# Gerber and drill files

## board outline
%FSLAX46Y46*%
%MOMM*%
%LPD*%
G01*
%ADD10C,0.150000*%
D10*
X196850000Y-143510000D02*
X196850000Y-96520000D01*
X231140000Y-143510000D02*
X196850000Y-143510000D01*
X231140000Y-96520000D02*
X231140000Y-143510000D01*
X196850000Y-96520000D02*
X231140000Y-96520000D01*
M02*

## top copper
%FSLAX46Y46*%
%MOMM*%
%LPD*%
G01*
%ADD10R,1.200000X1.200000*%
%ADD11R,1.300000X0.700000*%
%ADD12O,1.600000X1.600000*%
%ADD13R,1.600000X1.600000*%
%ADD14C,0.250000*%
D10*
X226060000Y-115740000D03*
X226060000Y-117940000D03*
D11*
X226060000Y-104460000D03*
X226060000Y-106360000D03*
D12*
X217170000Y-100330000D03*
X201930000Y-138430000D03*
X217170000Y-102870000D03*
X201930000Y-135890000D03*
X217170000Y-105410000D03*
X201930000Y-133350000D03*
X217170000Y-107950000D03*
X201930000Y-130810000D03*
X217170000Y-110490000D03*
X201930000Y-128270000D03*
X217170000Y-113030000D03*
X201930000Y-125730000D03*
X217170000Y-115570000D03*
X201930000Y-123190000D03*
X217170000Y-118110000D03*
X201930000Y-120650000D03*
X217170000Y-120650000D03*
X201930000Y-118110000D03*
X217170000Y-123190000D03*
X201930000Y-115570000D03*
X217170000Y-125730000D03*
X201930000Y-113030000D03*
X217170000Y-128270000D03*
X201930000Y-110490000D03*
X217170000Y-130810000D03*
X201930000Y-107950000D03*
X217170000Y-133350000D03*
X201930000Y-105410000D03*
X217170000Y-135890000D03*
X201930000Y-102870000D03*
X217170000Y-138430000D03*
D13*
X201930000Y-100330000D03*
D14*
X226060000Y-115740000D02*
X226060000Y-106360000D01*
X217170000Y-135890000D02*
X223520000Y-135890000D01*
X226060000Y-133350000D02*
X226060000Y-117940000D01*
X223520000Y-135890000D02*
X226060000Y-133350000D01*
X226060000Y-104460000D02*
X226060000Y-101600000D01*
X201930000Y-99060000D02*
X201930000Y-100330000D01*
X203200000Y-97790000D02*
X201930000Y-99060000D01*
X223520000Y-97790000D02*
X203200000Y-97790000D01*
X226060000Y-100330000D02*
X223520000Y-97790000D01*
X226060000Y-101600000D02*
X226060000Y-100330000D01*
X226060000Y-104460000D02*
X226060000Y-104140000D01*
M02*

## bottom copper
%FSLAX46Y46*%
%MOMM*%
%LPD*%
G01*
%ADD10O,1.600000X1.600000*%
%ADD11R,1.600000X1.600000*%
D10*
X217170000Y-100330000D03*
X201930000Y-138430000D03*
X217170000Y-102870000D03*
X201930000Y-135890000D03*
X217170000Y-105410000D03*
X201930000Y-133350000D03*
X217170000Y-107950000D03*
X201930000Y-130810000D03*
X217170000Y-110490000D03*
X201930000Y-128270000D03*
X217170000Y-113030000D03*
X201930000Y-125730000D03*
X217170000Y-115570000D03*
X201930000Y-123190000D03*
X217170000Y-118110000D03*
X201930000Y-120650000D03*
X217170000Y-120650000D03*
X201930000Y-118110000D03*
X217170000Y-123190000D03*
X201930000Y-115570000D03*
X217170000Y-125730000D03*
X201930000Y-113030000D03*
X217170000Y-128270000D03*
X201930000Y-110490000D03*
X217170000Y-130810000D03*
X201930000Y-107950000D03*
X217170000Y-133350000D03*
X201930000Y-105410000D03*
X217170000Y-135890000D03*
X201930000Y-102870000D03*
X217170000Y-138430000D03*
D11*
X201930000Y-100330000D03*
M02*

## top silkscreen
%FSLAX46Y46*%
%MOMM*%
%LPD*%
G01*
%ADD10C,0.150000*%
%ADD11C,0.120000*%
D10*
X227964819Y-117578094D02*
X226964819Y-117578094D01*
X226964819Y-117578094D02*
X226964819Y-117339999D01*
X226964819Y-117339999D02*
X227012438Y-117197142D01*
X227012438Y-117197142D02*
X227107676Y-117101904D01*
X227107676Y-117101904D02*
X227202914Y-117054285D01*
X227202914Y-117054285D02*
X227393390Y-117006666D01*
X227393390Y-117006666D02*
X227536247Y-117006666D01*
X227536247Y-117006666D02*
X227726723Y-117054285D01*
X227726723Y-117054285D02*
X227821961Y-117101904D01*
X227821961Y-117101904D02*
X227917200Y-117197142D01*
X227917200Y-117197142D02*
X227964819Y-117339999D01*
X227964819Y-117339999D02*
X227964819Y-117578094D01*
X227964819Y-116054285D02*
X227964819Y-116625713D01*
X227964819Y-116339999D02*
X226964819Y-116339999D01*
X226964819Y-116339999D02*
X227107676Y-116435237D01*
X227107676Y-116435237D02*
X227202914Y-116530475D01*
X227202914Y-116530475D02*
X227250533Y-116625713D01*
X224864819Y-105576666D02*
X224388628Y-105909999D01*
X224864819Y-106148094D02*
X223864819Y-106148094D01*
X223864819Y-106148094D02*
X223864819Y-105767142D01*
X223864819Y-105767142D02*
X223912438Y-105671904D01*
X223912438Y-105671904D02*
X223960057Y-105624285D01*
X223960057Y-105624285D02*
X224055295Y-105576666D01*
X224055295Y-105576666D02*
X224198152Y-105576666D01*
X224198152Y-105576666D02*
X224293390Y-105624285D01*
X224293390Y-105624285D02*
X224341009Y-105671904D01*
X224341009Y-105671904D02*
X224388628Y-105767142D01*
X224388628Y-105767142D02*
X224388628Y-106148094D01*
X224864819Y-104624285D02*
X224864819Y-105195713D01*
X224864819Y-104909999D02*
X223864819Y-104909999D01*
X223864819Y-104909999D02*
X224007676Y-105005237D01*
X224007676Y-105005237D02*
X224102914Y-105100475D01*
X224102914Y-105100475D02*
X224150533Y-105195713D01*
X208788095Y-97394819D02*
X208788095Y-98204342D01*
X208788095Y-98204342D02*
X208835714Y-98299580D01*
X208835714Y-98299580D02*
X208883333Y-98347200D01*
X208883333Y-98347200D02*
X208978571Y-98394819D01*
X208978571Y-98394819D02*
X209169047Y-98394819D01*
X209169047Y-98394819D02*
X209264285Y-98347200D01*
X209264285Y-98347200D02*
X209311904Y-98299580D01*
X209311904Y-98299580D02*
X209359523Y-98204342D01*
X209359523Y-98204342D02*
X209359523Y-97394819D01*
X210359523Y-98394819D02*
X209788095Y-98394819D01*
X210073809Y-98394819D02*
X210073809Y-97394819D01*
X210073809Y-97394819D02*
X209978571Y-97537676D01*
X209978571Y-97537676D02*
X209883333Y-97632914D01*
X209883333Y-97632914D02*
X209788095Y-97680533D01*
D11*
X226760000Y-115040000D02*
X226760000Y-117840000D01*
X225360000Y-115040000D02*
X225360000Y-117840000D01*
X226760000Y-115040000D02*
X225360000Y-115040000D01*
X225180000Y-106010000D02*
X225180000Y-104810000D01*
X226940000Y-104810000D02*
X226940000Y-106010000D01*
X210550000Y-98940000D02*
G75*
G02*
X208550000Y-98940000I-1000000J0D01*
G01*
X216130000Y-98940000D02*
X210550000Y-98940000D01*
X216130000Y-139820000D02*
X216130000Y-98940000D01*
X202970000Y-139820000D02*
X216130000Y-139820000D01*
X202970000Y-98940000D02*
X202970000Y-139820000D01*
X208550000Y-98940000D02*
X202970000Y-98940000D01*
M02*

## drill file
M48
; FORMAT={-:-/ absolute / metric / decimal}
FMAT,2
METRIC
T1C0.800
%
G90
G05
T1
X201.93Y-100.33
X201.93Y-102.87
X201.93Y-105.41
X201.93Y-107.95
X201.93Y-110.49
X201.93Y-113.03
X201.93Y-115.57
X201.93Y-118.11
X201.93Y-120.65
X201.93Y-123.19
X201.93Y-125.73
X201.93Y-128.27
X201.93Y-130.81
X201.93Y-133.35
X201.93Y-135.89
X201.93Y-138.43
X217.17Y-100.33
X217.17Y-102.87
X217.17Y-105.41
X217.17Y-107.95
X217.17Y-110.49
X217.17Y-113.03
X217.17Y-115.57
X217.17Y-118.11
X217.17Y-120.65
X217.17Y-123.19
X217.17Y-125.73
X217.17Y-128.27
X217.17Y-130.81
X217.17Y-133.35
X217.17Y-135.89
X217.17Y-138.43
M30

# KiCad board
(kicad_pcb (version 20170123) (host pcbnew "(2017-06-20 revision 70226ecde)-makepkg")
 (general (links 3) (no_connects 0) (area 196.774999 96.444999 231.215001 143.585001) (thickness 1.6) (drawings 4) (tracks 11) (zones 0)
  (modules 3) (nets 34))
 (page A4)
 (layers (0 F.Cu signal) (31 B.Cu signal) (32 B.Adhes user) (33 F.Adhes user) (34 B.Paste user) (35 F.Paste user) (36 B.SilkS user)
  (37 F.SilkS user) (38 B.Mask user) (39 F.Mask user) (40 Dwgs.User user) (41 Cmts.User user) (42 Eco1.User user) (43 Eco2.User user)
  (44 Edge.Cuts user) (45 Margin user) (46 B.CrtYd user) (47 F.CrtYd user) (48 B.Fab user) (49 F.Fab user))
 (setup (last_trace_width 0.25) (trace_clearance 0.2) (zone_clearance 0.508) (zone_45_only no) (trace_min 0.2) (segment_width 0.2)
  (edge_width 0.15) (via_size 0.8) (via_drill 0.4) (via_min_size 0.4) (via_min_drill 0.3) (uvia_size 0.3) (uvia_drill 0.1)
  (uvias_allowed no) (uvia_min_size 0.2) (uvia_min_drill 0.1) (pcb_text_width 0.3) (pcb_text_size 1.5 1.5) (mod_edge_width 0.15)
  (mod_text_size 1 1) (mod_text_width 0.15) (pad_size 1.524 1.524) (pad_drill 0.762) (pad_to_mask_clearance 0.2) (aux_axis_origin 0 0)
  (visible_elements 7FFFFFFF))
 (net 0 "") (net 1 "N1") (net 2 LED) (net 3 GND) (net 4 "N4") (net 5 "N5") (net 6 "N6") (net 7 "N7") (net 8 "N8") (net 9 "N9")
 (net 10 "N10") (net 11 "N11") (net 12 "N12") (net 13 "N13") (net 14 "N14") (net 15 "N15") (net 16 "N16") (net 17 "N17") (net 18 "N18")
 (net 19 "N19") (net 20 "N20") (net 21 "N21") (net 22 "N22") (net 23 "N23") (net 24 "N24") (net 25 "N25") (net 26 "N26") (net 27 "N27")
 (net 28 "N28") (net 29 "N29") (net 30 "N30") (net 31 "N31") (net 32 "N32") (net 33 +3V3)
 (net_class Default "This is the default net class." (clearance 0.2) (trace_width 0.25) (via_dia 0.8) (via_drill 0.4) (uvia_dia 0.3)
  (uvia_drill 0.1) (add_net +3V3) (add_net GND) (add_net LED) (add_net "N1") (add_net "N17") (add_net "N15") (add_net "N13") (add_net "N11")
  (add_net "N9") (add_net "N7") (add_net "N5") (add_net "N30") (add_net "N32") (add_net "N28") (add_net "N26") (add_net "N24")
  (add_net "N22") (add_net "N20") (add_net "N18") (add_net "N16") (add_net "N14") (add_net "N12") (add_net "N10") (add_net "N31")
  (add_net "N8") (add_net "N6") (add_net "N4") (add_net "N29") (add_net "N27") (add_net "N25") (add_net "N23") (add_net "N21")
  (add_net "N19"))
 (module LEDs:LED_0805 (layer F.Cu) (at 226.06 116.84 270)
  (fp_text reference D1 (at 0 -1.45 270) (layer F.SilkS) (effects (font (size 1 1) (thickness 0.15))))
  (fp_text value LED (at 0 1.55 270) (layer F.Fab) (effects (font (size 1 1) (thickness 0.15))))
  (fp_line (start -1.8 -0.7) (end 1 -0.7) (layer F.SilkS) (width 0.12))
  (fp_line (start -1.8 0.7) (end 1 0.7) (layer F.SilkS) (width 0.12))
  (fp_line (start -1.8 -0.7) (end -1.8 0.7) (layer F.SilkS) (width 0.12))
  (pad 1 smd rect (at -1.1 0 90) (size 1.2 1.2) (layers F.Cu F.Paste F.Mask) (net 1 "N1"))
  (pad 2 smd rect (at 1.1 0 90) (size 1.2 1.2) (layers F.Cu F.Paste F.Mask) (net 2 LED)))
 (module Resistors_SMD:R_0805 (layer F.Cu) (at 226.06 105.41 90)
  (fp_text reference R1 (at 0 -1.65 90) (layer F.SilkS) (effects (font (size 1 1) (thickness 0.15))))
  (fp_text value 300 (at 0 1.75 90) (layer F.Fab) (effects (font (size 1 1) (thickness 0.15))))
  (fp_line (start -0.6 -0.88) (end 0.6 -0.88) (layer F.SilkS) (width 0.12))
  (fp_line (start 0.6 0.88) (end -0.6 0.88) (layer F.SilkS) (width 0.12))
  (pad 2 smd rect (at 0.95 0 90) (size 0.7 1.3) (layers F.Cu F.Paste F.Mask) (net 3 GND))
  (pad 1 smd rect (at -0.95 0 90) (size 0.7 1.3) (layers F.Cu F.Paste F.Mask) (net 1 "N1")))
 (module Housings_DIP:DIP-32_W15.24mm (layer F.Cu) (at 201.93 100.33)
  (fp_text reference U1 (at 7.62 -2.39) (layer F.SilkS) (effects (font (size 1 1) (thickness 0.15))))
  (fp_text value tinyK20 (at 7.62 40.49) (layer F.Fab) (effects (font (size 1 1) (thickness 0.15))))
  (fp_arc (start 7.62 -1.39) (end 6.62 -1.39) (angle -180) (layer F.SilkS) (width 0.12))
  (fp_line (start 14.2 -1.39) (end 8.62 -1.39) (layer F.SilkS) (width 0.12))
  (fp_line (start 14.2 39.49) (end 14.2 -1.39) (layer F.SilkS) (width 0.12))
  (fp_line (start 1.04 39.49) (end 14.2 39.49) (layer F.SilkS) (width 0.12))
  (fp_line (start 1.04 -1.39) (end 1.04 39.49) (layer F.SilkS) (width 0.12))
  (fp_line (start 6.62 -1.39) (end 1.04 -1.39) (layer F.SilkS) (width 0.12))
  (pad 32 thru_hole oval (at 15.24 0) (size 1.6 1.6) (drill 0.8) (layers *.Cu *.Mask) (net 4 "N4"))
  (pad 16 thru_hole oval (at 0 38.1) (size 1.6 1.6) (drill 0.8) (layers *.Cu *.Mask) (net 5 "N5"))
  (pad 31 thru_hole oval (at 15.24 2.54) (size 1.6 1.6) (drill 0.8) (layers *.Cu *.Mask) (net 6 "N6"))
  (pad 15 thru_hole oval (at 0 35.56) (size 1.6 1.6) (drill 0.8) (layers *.Cu *.Mask) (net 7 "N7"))
  (pad 30 thru_hole oval (at 15.24 5.08) (size 1.6 1.6) (drill 0.8) (layers *.Cu *.Mask) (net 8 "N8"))
  (pad 14 thru_hole oval (at 0 33.02) (size 1.6 1.6) (drill 0.8) (layers *.Cu *.Mask) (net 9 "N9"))
  (pad 29 thru_hole oval (at 15.24 7.62) (size 1.6 1.6) (drill 0.8) (layers *.Cu *.Mask) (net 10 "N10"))
  (pad 13 thru_hole oval (at 0 30.48) (size 1.6 1.6) (drill 0.8) (layers *.Cu *.Mask) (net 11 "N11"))
  (pad 28 thru_hole oval (at 15.24 10.16) (size 1.6 1.6) (drill 0.8) (layers *.Cu *.Mask) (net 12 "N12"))
  (pad 12 thru_hole oval (at 0 27.94) (size 1.6 1.6) (drill 0.8) (layers *.Cu *.Mask) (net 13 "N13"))
  (pad 27 thru_hole oval (at 15.24 12.7) (size 1.6 1.6) (drill 0.8) (layers *.Cu *.Mask) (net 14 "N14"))
  (pad 11 thru_hole oval (at 0 25.4) (size 1.6 1.6) (drill 0.8) (layers *.Cu *.Mask) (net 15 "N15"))
  (pad 26 thru_hole oval (at 15.24 15.24) (size 1.6 1.6) (drill 0.8) (layers *.Cu *.Mask) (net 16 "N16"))
  (pad 10 thru_hole oval (at 0 22.86) (size 1.6 1.6) (drill 0.8) (layers *.Cu *.Mask) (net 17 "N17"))
  (pad 25 thru_hole oval (at 15.24 17.78) (size 1.6 1.6) (drill 0.8) (layers *.Cu *.Mask) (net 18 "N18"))
  (pad 9 thru_hole oval (at 0 20.32) (size 1.6 1.6) (drill 0.8) (layers *.Cu *.Mask) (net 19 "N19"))
  (pad 24 thru_hole oval (at 15.24 20.32) (size 1.6 1.6) (drill 0.8) (layers *.Cu *.Mask) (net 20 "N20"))
  (pad 8 thru_hole oval (at 0 17.78) (size 1.6 1.6) (drill 0.8) (layers *.Cu *.Mask) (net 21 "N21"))
  (pad 23 thru_hole oval (at 15.24 22.86) (size 1.6 1.6) (drill 0.8) (layers *.Cu *.Mask) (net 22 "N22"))
  (pad 7 thru_hole oval (at 0 15.24) (size 1.6 1.6) (drill 0.8) (layers *.Cu *.Mask) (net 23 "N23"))
  (pad 22 thru_hole oval (at 15.24 25.4) (size 1.6 1.6) (drill 0.8) (layers *.Cu *.Mask) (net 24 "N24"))
  (pad 6 thru_hole oval (at 0 12.7) (size 1.6 1.6) (drill 0.8) (layers *.Cu *.Mask) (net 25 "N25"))
  (pad 21 thru_hole oval (at 15.24 27.94) (size 1.6 1.6) (drill 0.8) (layers *.Cu *.Mask) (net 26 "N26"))
  (pad 5 thru_hole oval (at 0 10.16) (size 1.6 1.6) (drill 0.8) (layers *.Cu *.Mask) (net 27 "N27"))
  (pad 20 thru_hole oval (at 15.24 30.48) (size 1.6 1.6) (drill 0.8) (layers *.Cu *.Mask) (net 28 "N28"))
  (pad 4 thru_hole oval (at 0 7.62) (size 1.6 1.6) (drill 0.8) (layers *.Cu *.Mask) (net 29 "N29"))
  (pad 19 thru_hole oval (at 15.24 33.02) (size 1.6 1.6) (drill 0.8) (layers *.Cu *.Mask) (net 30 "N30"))
  (pad 3 thru_hole oval (at 0 5.08) (size 1.6 1.6) (drill 0.8) (layers *.Cu *.Mask) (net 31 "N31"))
  (pad 18 thru_hole oval (at 15.24 35.56) (size 1.6 1.6) (drill 0.8) (layers *.Cu *.Mask) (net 2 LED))
  (pad 2 thru_hole oval (at 0 2.54) (size 1.6 1.6) (drill 0.8) (layers *.Cu *.Mask) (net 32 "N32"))
  (pad 17 thru_hole oval (at 15.24 38.1) (size 1.6 1.6) (drill 0.8) (layers *.Cu *.Mask) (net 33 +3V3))
  (pad 1 thru_hole rect (at 0 0) (size 1.6 1.6) (drill 0.8) (layers *.Cu *.Mask) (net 3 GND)))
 (gr_line (start 196.85 143.51) (end 196.85 96.52) (angle 90) (layer Edge.Cuts) (width 0.15))
 (gr_line (start 231.14 143.51) (end 196.85 143.51) (angle 90) (layer Edge.Cuts) (width 0.15))
 (gr_line (start 231.14 96.52) (end 231.14 143.51) (angle 90) (layer Edge.Cuts) (width 0.15))
 (gr_line (start 196.85 96.52) (end 231.14 96.52) (angle 90) (layer Edge.Cuts) (width 0.15))
 (segment (start 226.06 115.74) (end 226.06 106.36) (width 0.25) (layer F.Cu) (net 1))
 (segment (start 217.17 135.89) (end 223.52 135.89) (width 0.25) (layer F.Cu) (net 2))
 (segment (start 226.06 133.35) (end 226.06 117.94) (width 0.25) (layer F.Cu) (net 2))
 (segment (start 223.52 135.89) (end 226.06 133.35) (width 0.25) (layer F.Cu) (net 2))
 (segment (start 226.06 104.46) (end 226.06 101.6) (width 0.25) (layer F.Cu) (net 3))
 (segment (start 201.93 99.06) (end 201.93 100.33) (width 0.25) (layer F.Cu) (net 3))
 (segment (start 203.2 97.79) (end 201.93 99.06) (width 0.25) (layer F.Cu) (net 3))
 (segment (start 223.52 97.79) (end 203.2 97.79) (width 0.25) (layer F.Cu) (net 3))
 (segment (start 226.06 100.33) (end 223.52 97.79) (width 0.25) (layer F.Cu) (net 3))
 (segment (start 226.06 101.6) (end 226.06 100.33) (width 0.25) (layer F.Cu) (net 3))
 (segment (start 226.06 104.46) (end 226.06 104.14) (width 0.25) (layer F.Cu) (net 3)))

